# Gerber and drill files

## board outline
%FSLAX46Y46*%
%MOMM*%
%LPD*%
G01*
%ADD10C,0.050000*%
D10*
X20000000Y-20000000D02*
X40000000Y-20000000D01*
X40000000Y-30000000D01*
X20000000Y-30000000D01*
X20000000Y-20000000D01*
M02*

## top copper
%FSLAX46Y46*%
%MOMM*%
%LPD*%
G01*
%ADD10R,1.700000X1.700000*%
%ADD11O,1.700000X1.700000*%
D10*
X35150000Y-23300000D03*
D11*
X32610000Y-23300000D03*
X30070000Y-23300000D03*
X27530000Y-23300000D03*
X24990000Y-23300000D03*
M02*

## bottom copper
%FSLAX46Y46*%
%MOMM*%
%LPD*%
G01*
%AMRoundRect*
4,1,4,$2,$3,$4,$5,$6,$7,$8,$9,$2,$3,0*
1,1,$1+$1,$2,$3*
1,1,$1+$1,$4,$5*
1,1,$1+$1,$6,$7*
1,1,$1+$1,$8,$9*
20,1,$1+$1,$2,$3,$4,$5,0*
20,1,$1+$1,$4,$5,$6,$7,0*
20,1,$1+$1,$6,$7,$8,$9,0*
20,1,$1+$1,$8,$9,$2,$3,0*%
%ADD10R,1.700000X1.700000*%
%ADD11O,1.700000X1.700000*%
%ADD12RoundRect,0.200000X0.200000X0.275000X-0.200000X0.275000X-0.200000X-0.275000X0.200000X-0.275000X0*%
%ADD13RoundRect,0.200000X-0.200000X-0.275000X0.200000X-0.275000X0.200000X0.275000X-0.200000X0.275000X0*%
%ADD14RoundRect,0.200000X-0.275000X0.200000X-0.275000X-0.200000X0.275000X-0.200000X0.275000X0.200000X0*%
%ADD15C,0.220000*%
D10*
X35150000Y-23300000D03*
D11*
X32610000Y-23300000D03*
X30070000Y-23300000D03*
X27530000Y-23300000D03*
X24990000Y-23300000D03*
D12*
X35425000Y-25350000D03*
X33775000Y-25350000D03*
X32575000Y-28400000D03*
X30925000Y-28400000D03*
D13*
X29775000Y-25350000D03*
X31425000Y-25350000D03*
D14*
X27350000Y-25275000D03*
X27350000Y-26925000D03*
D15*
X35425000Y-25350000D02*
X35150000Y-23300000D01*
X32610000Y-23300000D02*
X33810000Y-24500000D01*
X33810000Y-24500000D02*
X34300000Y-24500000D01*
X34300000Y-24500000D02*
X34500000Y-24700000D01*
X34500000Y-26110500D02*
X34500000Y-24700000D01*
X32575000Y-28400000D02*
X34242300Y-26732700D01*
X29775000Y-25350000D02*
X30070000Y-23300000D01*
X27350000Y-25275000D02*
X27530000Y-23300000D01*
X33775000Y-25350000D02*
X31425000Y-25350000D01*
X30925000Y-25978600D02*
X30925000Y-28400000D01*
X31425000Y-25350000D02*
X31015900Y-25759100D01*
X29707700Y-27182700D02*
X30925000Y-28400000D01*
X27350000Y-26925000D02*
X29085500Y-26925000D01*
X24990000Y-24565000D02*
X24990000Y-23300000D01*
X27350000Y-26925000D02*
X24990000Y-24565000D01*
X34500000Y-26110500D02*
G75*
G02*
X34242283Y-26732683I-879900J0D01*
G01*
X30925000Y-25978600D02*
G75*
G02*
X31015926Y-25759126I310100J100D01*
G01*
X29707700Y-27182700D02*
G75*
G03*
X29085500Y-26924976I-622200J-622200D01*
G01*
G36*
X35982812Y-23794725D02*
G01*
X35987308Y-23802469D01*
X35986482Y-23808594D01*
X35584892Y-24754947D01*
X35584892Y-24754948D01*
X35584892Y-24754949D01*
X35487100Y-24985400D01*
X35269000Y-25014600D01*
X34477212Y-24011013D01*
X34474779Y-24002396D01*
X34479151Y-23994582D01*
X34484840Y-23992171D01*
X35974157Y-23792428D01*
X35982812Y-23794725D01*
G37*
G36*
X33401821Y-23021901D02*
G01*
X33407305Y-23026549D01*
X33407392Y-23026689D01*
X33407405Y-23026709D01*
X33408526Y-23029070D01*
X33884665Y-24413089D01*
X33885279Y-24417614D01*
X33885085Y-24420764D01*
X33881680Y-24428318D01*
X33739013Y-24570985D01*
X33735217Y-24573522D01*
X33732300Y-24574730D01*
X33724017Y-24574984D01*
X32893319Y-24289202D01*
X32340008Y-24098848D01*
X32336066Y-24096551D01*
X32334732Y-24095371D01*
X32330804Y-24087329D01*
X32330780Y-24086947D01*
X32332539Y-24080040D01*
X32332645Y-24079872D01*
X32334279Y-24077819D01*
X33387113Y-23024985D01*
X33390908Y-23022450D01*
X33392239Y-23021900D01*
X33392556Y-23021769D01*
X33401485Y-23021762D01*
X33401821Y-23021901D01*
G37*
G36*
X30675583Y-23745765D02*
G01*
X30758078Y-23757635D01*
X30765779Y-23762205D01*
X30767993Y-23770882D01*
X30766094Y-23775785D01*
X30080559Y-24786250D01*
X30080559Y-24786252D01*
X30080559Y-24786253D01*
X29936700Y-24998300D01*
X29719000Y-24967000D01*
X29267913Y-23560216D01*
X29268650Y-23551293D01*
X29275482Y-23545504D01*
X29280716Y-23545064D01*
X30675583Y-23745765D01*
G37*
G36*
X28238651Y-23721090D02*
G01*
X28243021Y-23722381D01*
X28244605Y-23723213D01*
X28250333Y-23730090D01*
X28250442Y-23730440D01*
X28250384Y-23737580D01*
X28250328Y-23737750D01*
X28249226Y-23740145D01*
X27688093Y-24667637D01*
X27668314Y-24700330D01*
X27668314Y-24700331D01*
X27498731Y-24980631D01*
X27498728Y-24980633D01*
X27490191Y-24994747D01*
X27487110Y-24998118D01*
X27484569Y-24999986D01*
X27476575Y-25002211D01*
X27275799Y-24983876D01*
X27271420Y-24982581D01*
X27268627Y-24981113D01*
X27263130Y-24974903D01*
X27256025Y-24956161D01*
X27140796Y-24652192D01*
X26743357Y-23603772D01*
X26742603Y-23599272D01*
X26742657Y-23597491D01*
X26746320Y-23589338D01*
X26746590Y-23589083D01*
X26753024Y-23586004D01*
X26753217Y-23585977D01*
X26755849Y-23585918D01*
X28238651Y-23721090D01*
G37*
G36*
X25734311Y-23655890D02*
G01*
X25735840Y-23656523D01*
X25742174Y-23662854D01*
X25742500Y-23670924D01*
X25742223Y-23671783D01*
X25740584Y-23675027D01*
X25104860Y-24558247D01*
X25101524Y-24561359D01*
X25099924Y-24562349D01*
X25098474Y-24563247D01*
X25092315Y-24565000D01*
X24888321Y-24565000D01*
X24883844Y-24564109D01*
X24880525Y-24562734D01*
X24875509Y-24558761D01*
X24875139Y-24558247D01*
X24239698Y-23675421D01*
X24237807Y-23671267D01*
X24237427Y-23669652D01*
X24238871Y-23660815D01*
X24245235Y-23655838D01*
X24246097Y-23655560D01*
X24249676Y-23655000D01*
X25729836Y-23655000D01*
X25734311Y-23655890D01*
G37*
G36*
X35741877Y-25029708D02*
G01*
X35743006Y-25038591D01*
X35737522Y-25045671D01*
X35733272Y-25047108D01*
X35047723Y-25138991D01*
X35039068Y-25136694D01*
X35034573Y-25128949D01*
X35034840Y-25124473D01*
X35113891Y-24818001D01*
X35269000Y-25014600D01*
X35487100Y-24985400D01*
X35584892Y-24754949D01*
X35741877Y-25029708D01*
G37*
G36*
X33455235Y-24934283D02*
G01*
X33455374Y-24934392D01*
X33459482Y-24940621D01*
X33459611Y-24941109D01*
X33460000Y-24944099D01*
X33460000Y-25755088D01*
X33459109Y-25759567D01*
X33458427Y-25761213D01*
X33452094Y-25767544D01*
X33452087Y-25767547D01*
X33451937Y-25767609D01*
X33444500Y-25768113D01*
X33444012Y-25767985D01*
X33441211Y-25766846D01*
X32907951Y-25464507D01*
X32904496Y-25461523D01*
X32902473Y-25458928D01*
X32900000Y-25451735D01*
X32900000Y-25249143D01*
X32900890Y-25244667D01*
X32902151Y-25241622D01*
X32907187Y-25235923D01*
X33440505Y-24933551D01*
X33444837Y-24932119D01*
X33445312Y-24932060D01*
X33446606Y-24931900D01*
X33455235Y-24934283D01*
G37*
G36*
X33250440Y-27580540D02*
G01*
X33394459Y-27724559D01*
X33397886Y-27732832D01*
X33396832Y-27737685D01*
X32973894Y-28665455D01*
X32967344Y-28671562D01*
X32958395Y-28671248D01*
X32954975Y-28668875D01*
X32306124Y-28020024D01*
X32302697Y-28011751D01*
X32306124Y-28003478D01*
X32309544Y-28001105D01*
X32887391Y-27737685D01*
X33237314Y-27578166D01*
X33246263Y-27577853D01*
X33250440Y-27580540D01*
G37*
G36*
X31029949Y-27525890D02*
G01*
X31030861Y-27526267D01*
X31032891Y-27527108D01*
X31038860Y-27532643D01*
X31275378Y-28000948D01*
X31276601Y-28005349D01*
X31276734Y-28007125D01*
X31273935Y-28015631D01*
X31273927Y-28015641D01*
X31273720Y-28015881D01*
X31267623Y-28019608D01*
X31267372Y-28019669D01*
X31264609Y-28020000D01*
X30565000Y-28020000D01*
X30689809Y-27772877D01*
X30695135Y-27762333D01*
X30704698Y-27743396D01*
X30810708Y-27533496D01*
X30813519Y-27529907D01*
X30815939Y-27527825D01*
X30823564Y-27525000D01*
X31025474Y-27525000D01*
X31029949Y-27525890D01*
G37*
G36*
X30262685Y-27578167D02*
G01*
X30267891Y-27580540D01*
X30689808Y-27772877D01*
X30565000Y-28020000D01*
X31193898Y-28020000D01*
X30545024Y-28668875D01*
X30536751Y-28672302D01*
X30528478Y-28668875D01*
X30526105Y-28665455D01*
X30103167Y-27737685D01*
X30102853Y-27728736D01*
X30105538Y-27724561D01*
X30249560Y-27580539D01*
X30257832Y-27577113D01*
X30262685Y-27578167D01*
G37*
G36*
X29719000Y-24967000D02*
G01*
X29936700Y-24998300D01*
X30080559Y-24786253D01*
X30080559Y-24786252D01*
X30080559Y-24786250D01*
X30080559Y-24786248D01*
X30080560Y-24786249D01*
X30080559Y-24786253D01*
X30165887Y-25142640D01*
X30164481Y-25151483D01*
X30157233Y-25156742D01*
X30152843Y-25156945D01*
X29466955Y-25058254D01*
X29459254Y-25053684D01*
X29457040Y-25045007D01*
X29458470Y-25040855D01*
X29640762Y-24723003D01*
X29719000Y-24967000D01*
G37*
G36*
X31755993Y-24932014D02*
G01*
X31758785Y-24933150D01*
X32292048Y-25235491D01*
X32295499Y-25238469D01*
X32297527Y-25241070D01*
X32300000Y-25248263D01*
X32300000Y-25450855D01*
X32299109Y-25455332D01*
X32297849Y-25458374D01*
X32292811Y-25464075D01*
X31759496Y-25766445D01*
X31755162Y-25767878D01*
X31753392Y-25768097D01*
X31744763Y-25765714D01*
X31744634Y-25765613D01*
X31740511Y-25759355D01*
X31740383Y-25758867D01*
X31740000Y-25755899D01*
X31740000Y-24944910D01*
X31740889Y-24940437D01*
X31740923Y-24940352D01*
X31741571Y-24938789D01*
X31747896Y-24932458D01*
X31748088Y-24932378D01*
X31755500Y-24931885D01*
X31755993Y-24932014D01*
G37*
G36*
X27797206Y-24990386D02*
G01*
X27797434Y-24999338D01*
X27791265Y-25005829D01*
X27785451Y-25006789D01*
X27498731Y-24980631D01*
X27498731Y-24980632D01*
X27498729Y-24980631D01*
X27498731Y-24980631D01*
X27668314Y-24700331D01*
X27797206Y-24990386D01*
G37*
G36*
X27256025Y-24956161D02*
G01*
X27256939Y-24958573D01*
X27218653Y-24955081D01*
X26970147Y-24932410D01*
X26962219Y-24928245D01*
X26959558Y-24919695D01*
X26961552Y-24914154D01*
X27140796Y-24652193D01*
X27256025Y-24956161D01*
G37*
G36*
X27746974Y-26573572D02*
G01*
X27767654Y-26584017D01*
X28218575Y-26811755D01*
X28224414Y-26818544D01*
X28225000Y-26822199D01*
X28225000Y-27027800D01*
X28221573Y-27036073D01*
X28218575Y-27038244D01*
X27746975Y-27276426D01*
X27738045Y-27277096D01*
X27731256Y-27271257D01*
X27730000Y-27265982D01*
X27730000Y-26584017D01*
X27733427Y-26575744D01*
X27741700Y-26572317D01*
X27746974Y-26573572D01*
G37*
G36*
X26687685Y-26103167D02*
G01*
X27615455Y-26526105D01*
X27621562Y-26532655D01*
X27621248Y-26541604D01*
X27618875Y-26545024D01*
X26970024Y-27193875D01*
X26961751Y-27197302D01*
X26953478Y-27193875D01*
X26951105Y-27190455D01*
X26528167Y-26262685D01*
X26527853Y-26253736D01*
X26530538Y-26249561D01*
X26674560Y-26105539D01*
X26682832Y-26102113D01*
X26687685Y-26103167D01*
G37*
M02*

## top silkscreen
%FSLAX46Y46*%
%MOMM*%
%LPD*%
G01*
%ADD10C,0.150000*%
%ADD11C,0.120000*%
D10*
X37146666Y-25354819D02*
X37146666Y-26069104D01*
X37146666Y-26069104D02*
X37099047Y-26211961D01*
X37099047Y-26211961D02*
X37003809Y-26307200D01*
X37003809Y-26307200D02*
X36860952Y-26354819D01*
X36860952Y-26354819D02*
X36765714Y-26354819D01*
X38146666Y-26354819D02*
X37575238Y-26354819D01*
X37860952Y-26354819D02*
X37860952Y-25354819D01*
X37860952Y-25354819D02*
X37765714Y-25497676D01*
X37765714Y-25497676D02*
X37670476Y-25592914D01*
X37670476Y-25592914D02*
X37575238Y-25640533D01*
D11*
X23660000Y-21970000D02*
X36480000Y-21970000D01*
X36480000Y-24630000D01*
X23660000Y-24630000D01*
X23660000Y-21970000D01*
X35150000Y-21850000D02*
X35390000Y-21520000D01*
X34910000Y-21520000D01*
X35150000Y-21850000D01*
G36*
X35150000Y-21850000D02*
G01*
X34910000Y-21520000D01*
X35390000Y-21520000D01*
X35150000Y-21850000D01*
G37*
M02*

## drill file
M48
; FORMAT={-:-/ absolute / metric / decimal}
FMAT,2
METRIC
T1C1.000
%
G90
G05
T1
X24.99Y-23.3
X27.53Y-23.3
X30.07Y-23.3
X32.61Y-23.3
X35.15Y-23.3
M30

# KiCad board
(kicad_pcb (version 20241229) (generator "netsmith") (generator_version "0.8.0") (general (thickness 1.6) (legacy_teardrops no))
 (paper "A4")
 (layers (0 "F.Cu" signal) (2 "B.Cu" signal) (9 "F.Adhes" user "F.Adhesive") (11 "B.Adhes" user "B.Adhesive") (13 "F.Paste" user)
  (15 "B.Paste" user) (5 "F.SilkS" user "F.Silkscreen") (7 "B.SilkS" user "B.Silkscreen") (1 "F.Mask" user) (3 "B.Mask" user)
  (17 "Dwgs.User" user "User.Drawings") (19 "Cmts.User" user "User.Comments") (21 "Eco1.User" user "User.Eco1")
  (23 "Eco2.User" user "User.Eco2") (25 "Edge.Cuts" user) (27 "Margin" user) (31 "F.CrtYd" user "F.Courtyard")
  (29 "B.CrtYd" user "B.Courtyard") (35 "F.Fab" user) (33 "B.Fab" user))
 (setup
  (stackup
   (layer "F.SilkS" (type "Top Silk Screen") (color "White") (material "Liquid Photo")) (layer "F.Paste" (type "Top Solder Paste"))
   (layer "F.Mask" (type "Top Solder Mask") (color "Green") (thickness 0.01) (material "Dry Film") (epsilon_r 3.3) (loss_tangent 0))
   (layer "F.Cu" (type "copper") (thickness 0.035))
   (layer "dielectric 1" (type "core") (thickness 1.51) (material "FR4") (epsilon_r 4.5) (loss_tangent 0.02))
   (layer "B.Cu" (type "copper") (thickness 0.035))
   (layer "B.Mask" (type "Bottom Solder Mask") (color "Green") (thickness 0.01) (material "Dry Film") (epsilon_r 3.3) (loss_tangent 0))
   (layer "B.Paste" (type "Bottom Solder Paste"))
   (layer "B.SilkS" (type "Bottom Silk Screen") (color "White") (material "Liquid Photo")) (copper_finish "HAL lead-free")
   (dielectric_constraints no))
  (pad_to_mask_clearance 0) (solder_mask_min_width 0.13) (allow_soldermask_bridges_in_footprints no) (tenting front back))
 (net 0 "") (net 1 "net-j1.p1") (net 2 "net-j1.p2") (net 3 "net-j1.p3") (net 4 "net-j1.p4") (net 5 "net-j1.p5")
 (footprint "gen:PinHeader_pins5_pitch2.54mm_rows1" (layer "F.Cu") (at 35.15 23.3 270)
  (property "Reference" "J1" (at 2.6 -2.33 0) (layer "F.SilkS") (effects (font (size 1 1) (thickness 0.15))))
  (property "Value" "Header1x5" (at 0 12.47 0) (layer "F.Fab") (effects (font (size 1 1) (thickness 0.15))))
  (pad "1" thru_hole rect (at 0 0 270) (size 1.7 1.7) (drill 1) (layers "*.Cu" "*.Mask") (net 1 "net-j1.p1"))
  (pad "2" thru_hole oval (at 0 2.54 270) (size 1.7 1.7) (drill 1) (layers "*.Cu" "*.Mask") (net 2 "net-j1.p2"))
  (pad "3" thru_hole oval (at 0 5.08 270) (size 1.7 1.7) (drill 1) (layers "*.Cu" "*.Mask") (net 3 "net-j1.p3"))
  (pad "4" thru_hole oval (at 0 7.62 270) (size 1.7 1.7) (drill 1) (layers "*.Cu" "*.Mask") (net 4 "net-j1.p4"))
  (pad "5" thru_hole oval (at 0 10.16 270) (size 1.7 1.7) (drill 1) (layers "*.Cu" "*.Mask") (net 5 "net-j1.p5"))
  (fp_rect (start -1.33 -1.33) (end 1.33 11.49) (stroke (width 0.12) (type solid)) (fill no) (layer "F.SilkS"))
  (fp_poly (pts (xy -1.45 0) (xy -1.78 -0.24) (xy -1.78 0.24)) (stroke (width 0.12) (type solid)) (fill solid) (layer "F.SilkS")))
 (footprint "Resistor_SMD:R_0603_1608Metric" (layer "B.Cu") (at 34.6 25.35 180)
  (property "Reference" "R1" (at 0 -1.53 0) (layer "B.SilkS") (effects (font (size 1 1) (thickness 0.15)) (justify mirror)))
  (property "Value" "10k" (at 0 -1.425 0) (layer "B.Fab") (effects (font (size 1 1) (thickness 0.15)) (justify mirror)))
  (pad "1" smd roundrect (at -0.825 0 180) (size 0.8 0.95) (layers "B.Cu" "B.Mask" "B.Paste") (roundrect_rratio 0.25) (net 1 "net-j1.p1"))
  (pad "2" smd roundrect (at 0.825 0 180) (size 0.8 0.95) (layers "B.Cu" "B.Mask" "B.Paste") (roundrect_rratio 0.25) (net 5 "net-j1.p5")))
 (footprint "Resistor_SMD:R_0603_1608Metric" (layer "B.Cu") (at 31.75 28.4 180)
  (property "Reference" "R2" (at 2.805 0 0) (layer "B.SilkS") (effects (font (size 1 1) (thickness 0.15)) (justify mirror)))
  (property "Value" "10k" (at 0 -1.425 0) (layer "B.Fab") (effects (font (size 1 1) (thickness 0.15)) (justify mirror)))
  (pad "1" smd roundrect (at -0.825 0 180) (size 0.8 0.95) (layers "B.Cu" "B.Mask" "B.Paste") (roundrect_rratio 0.25) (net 2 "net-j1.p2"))
  (pad "2" smd roundrect (at 0.825 0 180) (size 0.8 0.95) (layers "B.Cu" "B.Mask" "B.Paste") (roundrect_rratio 0.25) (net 5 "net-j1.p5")))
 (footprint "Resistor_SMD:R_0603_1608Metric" (layer "B.Cu") (at 30.6 25.35)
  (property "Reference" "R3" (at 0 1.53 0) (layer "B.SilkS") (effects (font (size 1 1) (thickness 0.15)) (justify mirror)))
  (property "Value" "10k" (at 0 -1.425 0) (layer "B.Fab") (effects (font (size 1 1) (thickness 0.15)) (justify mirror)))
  (pad "1" smd roundrect (at -0.825 0) (size 0.8 0.95) (layers "B.Cu" "B.Mask" "B.Paste") (roundrect_rratio 0.25) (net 3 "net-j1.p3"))
  (pad "2" smd roundrect (at 0.825 0) (size 0.8 0.95) (layers "B.Cu" "B.Mask" "B.Paste") (roundrect_rratio 0.25) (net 5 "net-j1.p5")))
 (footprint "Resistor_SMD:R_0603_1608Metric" (layer "B.Cu") (at 27.35 26.1 270)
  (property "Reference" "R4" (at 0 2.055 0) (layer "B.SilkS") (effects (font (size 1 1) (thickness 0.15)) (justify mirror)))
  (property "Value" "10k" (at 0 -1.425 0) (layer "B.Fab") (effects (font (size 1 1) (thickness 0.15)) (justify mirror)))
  (pad "1" smd roundrect (at -0.825 0 270) (size 0.8 0.95) (layers "B.Cu" "B.Mask" "B.Paste") (roundrect_rratio 0.25) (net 4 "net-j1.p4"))
  (pad "2" smd roundrect (at 0.825 0 270) (size 0.8 0.95) (layers "B.Cu" "B.Mask" "B.Paste") (roundrect_rratio 0.25) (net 5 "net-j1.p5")))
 (segment (start 35.425 25.35) (end 35.15 23.3) (width 0.22) (layer "B.Cu") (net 1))
 (segment (start 32.61 23.3) (end 33.81 24.5) (width 0.22) (layer "B.Cu") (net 2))
 (segment (start 33.81 24.5) (end 34.3 24.5) (width 0.22) (layer "B.Cu") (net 2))
 (segment (start 34.3 24.5) (end 34.5 24.7) (width 0.22) (layer "B.Cu") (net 2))
 (segment (start 34.5 26.1105) (end 34.5 24.7) (width 0.22) (layer "B.Cu") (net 2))
 (segment (start 32.575 28.4) (end 34.2423 26.7327) (width 0.22) (layer "B.Cu") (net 2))
 (segment (start 29.775 25.35) (end 30.07 23.3) (width 0.22) (layer "B.Cu") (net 3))
 (segment (start 27.35 25.275) (end 27.53 23.3) (width 0.22) (layer "B.Cu") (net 4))
 (segment (start 33.775 25.35) (end 31.425 25.35) (width 0.22) (layer "B.Cu") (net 5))
 (segment (start 30.925 25.9786) (end 30.925 28.4) (width 0.22) (layer "B.Cu") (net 5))
 (segment (start 31.425 25.35) (end 31.0159 25.7591) (width 0.22) (layer "B.Cu") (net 5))
 (segment (start 29.7077 27.1827) (end 30.925 28.4) (width 0.22) (layer "B.Cu") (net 5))
 (segment (start 27.35 26.925) (end 29.0855 26.925) (width 0.22) (layer "B.Cu") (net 5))
 (segment (start 24.99 24.565) (end 24.99 23.3) (width 0.22) (layer "B.Cu") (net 5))
 (segment (start 27.35 26.925) (end 24.99 24.565) (width 0.22) (layer "B.Cu") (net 5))
 (arc (start 34.5 26.1105) (mid 34.433 26.4473) (end 34.2423 26.7327) (width 0.22) (layer "B.Cu") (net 2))
 (arc (start 30.925 25.9786) (mid 30.9486 25.8598) (end 31.0159 25.7591) (width 0.22) (layer "B.Cu") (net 5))
 (arc (start 29.7077 27.1827) (mid 29.4223 26.992) (end 29.0855 26.925) (width 0.22) (layer "B.Cu") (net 5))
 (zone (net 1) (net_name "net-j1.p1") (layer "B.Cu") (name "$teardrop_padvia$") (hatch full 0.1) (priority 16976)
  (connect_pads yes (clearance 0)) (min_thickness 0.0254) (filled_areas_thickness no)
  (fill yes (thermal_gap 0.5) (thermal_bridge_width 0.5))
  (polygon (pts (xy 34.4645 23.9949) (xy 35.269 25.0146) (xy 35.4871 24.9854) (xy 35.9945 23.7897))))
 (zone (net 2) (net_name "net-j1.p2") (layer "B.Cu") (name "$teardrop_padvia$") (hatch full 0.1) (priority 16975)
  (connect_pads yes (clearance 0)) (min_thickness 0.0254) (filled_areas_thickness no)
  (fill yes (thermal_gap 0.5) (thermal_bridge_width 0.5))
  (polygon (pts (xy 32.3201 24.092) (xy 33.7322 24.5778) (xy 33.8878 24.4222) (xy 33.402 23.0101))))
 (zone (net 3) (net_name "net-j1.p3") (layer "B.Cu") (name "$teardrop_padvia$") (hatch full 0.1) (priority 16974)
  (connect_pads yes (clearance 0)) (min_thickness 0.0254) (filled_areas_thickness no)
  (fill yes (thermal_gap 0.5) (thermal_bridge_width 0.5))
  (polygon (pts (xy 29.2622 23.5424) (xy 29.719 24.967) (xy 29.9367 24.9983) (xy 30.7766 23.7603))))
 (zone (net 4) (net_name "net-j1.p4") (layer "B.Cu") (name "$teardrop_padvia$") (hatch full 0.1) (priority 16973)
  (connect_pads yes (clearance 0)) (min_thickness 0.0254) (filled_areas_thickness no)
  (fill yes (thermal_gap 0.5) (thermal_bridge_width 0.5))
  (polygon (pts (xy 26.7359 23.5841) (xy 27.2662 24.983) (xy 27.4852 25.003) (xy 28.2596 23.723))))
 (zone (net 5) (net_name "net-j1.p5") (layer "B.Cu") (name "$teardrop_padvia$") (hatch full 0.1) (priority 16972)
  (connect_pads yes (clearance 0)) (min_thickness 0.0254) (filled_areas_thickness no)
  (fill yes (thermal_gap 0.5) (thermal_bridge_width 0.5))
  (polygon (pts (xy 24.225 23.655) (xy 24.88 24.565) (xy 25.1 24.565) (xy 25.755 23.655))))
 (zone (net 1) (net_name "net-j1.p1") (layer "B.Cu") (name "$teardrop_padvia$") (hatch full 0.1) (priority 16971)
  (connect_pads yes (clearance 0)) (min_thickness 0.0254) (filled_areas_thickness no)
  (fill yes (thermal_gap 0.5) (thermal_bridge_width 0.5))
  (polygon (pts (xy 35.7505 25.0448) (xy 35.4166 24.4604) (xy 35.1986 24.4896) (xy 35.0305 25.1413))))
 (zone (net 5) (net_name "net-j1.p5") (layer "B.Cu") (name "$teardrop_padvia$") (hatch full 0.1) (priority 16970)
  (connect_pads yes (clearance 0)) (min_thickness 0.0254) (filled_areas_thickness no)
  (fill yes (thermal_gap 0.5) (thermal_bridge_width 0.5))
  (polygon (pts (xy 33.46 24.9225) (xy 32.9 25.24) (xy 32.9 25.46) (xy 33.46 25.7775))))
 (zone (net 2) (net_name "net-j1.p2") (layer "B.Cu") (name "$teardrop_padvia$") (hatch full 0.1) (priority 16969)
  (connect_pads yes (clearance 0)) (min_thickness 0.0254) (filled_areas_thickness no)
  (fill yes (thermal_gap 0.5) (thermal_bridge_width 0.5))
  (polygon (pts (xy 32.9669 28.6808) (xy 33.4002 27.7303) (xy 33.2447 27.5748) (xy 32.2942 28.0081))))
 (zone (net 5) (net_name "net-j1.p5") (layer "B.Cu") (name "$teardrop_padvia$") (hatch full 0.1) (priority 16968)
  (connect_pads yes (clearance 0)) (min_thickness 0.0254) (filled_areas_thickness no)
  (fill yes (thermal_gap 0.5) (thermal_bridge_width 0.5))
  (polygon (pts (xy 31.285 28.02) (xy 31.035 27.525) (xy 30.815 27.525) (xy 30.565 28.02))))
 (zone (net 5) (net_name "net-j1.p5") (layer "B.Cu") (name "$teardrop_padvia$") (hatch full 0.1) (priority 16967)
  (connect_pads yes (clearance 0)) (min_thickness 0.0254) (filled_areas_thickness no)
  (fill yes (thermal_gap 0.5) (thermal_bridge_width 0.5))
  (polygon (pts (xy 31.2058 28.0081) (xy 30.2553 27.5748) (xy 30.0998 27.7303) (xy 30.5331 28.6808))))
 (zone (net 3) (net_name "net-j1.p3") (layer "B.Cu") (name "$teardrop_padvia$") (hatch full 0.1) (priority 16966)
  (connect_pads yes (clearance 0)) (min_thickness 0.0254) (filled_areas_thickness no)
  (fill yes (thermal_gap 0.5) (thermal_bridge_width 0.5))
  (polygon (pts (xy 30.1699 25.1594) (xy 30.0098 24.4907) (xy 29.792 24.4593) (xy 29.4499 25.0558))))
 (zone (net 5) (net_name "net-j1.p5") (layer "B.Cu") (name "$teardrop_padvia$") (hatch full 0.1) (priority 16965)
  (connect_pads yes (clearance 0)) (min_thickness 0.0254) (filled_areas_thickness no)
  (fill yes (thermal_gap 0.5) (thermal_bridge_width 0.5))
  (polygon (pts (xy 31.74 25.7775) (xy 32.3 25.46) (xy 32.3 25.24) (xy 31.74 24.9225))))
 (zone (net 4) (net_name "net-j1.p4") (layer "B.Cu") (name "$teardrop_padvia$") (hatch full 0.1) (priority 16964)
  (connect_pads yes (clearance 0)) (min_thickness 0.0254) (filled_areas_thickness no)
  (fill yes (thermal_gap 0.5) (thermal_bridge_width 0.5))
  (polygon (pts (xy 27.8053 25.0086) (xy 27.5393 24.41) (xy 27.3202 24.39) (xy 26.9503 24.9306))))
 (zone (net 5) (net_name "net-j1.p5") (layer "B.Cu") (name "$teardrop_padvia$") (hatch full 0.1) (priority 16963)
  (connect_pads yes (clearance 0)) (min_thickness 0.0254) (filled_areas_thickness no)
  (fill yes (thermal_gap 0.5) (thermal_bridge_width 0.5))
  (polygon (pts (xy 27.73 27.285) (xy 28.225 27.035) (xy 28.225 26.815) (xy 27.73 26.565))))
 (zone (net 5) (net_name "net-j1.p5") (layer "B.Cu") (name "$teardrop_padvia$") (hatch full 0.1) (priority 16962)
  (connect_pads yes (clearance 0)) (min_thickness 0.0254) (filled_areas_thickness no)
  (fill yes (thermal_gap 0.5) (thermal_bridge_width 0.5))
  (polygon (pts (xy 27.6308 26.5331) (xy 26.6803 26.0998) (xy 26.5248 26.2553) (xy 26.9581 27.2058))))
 (gr_rect (start 20 20) (end 40 30) (stroke (width 0.05) (type default)) (fill no) (layer "Edge.Cuts")))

